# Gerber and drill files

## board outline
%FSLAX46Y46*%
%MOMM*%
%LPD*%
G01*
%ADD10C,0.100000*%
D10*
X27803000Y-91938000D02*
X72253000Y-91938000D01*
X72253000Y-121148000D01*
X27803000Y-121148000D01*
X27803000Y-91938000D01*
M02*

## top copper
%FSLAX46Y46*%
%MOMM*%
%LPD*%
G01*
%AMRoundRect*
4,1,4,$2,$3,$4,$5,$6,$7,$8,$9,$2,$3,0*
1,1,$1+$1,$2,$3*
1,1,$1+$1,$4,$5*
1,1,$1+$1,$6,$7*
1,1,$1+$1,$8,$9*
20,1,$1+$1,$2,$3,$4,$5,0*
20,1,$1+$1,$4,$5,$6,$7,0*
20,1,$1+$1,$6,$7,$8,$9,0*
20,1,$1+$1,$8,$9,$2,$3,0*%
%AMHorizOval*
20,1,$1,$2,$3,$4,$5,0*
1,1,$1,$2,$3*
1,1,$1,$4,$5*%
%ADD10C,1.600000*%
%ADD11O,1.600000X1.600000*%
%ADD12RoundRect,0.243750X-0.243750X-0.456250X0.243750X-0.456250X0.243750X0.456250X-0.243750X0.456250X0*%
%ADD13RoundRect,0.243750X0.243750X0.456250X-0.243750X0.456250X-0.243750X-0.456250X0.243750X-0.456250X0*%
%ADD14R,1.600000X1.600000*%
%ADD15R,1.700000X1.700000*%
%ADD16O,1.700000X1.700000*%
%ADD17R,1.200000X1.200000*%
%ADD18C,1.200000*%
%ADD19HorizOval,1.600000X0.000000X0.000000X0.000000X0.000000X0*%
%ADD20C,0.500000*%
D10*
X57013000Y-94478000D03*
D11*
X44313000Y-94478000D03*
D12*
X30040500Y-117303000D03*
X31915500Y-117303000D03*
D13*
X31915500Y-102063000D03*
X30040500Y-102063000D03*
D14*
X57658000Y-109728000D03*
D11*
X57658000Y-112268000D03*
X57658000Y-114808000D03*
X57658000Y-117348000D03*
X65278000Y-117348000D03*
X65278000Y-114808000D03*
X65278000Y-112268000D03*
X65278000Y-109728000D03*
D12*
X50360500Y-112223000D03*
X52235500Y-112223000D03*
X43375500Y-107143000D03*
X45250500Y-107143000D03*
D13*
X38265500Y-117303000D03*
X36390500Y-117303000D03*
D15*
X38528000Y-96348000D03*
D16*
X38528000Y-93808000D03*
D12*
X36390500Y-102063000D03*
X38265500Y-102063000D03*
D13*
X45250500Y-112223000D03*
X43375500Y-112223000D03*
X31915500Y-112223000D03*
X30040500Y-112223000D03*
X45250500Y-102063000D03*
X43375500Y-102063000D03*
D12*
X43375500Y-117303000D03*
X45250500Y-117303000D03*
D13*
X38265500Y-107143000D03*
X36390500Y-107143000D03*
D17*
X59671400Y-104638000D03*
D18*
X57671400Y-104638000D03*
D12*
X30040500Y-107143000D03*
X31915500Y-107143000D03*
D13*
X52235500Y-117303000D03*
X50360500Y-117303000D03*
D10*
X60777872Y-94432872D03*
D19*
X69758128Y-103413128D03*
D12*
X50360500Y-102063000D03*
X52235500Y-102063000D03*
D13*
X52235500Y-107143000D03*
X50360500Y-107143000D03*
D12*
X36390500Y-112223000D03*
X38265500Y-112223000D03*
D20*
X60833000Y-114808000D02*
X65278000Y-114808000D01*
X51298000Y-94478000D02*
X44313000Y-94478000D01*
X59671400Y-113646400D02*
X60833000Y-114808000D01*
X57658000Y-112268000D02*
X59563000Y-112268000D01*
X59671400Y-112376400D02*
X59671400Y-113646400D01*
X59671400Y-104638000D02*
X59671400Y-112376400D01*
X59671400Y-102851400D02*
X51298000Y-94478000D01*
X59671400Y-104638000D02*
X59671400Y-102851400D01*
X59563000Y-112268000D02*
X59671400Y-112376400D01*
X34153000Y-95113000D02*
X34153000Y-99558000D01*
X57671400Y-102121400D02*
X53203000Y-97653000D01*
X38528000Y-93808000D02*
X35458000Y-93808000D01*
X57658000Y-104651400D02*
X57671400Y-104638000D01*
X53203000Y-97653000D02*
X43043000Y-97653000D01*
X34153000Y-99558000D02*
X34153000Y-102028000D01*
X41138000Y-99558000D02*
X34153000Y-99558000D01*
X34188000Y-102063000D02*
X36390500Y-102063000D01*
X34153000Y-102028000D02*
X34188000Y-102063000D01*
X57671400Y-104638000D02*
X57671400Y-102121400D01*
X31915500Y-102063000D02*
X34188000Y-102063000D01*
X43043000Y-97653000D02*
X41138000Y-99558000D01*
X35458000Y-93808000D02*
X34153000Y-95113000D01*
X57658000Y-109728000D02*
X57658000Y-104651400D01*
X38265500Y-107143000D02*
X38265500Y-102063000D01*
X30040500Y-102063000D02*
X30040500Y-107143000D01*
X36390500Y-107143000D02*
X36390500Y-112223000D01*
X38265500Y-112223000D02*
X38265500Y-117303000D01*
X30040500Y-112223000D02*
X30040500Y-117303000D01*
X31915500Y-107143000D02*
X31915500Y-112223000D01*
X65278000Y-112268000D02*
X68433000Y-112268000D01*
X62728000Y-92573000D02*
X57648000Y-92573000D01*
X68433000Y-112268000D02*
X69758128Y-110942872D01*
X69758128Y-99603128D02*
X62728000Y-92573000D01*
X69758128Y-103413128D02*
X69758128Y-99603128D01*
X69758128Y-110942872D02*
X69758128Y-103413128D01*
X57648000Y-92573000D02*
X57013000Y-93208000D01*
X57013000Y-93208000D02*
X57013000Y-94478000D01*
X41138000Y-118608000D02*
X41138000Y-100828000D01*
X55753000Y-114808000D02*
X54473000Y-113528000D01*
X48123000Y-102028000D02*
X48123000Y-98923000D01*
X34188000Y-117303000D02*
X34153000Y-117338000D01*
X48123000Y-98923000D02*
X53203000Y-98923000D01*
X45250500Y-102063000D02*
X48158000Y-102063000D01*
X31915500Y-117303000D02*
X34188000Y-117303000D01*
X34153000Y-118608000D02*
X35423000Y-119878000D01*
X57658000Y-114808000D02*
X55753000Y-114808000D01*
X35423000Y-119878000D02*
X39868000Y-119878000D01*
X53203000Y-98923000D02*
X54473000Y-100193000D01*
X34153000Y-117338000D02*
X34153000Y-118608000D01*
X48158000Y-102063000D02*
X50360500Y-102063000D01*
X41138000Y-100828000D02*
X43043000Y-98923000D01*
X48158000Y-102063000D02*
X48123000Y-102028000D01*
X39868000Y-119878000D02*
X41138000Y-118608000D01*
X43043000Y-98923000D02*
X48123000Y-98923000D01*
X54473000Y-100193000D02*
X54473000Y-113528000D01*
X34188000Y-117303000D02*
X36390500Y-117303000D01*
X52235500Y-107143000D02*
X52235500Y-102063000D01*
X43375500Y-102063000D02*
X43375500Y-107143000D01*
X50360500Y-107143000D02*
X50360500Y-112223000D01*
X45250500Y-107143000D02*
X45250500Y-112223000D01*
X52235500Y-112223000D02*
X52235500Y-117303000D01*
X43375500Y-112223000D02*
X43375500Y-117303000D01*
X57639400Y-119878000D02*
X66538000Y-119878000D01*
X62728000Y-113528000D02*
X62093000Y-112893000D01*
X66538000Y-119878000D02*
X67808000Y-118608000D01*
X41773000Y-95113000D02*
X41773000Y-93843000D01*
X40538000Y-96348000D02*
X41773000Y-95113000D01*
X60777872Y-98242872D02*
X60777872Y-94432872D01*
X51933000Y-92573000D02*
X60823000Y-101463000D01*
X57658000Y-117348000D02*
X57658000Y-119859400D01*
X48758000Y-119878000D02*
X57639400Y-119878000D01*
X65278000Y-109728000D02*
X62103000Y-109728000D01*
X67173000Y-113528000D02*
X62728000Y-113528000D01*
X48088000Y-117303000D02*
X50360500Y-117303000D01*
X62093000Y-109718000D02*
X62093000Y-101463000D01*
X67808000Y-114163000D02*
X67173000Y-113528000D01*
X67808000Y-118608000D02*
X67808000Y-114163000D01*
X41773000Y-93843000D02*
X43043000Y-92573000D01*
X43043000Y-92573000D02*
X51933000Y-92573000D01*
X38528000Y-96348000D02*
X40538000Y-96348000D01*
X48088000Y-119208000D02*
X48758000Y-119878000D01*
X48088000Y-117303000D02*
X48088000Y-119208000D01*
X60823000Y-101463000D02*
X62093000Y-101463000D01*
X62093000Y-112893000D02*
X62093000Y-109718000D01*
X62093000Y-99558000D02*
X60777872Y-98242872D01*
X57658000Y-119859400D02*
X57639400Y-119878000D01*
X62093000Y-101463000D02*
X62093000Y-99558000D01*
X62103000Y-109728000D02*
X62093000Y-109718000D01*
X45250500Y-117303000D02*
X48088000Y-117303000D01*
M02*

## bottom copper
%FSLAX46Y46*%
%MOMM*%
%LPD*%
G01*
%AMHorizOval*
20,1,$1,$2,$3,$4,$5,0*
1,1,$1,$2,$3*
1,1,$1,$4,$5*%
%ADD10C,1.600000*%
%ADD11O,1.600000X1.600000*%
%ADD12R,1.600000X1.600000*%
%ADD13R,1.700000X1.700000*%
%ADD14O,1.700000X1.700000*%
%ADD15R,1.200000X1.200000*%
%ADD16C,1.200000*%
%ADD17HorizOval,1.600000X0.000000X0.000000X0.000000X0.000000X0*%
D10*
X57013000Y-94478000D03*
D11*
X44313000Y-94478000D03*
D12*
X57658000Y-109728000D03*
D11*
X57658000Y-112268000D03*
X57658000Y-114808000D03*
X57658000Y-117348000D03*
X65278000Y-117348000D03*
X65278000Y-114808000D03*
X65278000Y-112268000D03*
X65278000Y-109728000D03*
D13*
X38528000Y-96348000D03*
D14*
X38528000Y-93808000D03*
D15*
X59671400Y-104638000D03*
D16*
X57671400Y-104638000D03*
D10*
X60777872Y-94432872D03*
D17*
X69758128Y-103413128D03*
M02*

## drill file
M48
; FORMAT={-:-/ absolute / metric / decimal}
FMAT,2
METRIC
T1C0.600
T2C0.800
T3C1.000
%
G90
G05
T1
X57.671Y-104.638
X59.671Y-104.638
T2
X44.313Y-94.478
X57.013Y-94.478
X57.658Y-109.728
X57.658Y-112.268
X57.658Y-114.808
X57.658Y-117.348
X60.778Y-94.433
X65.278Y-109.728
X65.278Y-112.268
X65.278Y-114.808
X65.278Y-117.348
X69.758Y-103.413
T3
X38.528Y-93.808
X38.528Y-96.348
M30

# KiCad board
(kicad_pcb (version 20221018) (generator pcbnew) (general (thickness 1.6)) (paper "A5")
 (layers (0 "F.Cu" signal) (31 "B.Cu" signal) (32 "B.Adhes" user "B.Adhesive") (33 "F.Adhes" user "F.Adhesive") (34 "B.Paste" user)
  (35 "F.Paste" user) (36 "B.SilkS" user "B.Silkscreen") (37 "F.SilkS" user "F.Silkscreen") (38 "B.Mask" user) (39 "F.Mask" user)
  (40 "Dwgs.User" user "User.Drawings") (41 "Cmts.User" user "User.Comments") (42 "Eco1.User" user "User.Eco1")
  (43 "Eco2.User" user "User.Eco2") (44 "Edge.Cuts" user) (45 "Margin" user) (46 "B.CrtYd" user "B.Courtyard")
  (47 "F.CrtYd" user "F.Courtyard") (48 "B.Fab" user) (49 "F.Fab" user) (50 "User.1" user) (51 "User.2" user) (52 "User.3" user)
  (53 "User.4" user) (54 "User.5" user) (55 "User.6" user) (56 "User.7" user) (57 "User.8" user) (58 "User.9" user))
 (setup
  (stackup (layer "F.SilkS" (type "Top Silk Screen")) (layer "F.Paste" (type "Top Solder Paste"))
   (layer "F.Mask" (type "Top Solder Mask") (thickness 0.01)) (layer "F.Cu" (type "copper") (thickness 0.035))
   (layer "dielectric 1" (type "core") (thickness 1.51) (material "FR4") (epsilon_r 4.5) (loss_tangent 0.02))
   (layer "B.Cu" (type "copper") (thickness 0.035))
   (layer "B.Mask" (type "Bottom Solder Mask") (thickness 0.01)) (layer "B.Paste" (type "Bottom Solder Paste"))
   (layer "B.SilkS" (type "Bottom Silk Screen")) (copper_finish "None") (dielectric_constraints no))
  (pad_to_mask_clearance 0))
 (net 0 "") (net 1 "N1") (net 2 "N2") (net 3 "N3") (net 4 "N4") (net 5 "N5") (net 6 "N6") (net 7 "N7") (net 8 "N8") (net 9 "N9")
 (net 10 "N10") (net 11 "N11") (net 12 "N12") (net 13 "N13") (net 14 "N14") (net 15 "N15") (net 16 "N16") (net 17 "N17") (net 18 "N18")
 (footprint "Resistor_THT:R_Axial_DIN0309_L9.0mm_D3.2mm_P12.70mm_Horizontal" (layer "F.Cu") (at 57.013 94.478 180)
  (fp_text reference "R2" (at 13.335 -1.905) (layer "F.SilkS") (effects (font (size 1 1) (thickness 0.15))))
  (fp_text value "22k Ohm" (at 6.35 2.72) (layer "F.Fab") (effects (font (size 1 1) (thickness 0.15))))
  (pad "1" thru_hole circle (at 0 0 180) (size 1.6 1.6) (drill 0.8) (layers "*.Cu" "*.Mask") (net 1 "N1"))
  (pad "2" thru_hole oval (at 12.7 0 180) (size 1.6 1.6) (drill 0.8) (layers "*.Cu" "*.Mask") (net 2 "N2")))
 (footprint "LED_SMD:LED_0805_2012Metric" (layer "F.Cu") (at 30.978 117.303)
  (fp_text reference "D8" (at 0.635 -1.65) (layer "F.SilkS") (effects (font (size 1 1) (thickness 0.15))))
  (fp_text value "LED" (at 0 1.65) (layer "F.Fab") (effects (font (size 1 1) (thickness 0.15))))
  (pad "1" smd roundrect (at -0.9375 0) (size 0.975 1.4) (layers "F.Cu" "F.Paste" "F.Mask") (roundrect_rratio 0.25) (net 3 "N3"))
  (pad "2" smd roundrect (at 0.9375 0) (size 0.975 1.4) (layers "F.Cu" "F.Paste" "F.Mask") (roundrect_rratio 0.25) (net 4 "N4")))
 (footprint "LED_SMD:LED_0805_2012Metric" (layer "F.Cu") (at 30.978 102.063 180)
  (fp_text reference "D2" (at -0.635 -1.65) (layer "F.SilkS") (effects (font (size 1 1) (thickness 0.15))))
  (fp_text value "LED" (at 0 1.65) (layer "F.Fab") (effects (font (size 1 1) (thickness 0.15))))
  (pad "1" smd roundrect (at -0.9375 0 180) (size 0.975 1.4) (layers "F.Cu" "F.Paste" "F.Mask") (roundrect_rratio 0.25) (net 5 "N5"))
  (pad "2" smd roundrect (at 0.9375 0 180) (size 0.975 1.4) (layers "F.Cu" "F.Paste" "F.Mask") (roundrect_rratio 0.25) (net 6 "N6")))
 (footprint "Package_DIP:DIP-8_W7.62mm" (layer "F.Cu") (at 57.658 109.728)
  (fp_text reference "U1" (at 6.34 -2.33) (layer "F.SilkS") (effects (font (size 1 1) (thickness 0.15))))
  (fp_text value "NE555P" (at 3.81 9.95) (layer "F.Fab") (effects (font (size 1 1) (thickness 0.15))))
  (pad "1" thru_hole rect (at 0 0) (size 1.6 1.6) (drill 0.8) (layers "*.Cu" "*.Mask") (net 5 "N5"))
  (pad "2" thru_hole oval (at 0 2.54) (size 1.6 1.6) (drill 0.8) (layers "*.Cu" "*.Mask") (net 2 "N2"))
  (pad "3" thru_hole oval (at 0 5.08) (size 1.6 1.6) (drill 0.8) (layers "*.Cu" "*.Mask") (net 4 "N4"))
  (pad "4" thru_hole oval (at 0 7.62) (size 1.6 1.6) (drill 0.8) (layers "*.Cu" "*.Mask") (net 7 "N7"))
  (pad "5" thru_hole oval (at 7.62 7.62) (size 1.6 1.6) (drill 0.8) (layers "*.Cu" "*.Mask") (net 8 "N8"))
  (pad "6" thru_hole oval (at 7.62 5.08) (size 1.6 1.6) (drill 0.8) (layers "*.Cu" "*.Mask") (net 2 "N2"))
  (pad "7" thru_hole oval (at 7.62 2.54) (size 1.6 1.6) (drill 0.8) (layers "*.Cu" "*.Mask") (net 1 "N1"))
  (pad "8" thru_hole oval (at 7.62 0) (size 1.6 1.6) (drill 0.8) (layers "*.Cu" "*.Mask") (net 7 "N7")))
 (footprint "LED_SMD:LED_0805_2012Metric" (layer "F.Cu") (at 51.298 112.223)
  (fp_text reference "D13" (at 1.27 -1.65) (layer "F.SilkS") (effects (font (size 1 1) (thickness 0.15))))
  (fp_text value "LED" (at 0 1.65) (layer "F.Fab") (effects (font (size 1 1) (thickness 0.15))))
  (pad "1" smd roundrect (at -0.9375 0) (size 0.975 1.4) (layers "F.Cu" "F.Paste" "F.Mask") (roundrect_rratio 0.25) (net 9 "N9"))
  (pad "2" smd roundrect (at 0.9375 0) (size 0.975 1.4) (layers "F.Cu" "F.Paste" "F.Mask") (roundrect_rratio 0.25) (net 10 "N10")))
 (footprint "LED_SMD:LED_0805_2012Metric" (layer "F.Cu") (at 44.313 107.143)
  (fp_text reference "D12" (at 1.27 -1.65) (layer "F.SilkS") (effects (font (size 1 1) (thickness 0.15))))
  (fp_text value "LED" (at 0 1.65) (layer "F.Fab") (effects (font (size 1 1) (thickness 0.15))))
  (pad "1" smd roundrect (at -0.9375 0) (size 0.975 1.4) (layers "F.Cu" "F.Paste" "F.Mask") (roundrect_rratio 0.25) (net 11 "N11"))
  (pad "2" smd roundrect (at 0.9375 0) (size 0.975 1.4) (layers "F.Cu" "F.Paste" "F.Mask") (roundrect_rratio 0.25) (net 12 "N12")))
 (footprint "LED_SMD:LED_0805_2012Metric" (layer "F.Cu") (at 37.328 117.303 180)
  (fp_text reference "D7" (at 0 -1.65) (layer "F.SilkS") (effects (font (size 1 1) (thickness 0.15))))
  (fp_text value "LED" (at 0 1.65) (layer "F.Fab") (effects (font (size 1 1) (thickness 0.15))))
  (pad "1" smd roundrect (at -0.9375 0 180) (size 0.975 1.4) (layers "F.Cu" "F.Paste" "F.Mask") (roundrect_rratio 0.25) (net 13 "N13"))
  (pad "2" smd roundrect (at 0.9375 0 180) (size 0.975 1.4) (layers "F.Cu" "F.Paste" "F.Mask") (roundrect_rratio 0.25) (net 4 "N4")))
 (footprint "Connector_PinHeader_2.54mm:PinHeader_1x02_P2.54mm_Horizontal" (layer "F.Cu") (at 38.528 96.348 180)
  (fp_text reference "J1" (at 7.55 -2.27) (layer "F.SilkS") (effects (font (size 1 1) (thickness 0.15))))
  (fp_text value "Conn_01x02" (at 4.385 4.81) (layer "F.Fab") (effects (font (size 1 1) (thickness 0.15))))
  (pad "1" thru_hole rect (at 0 0 180) (size 1.7 1.7) (drill 1) (layers "*.Cu" "*.Mask") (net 7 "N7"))
  (pad "2" thru_hole oval (at 0 2.54 180) (size 1.7 1.7) (drill 1) (layers "*.Cu" "*.Mask") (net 5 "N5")))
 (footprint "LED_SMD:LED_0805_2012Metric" (layer "F.Cu") (at 37.328 102.063)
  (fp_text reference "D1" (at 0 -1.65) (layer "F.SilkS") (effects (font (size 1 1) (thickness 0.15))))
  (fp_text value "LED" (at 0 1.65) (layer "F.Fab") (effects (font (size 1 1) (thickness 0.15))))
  (pad "1" smd roundrect (at -0.9375 0) (size 0.975 1.4) (layers "F.Cu" "F.Paste" "F.Mask") (roundrect_rratio 0.25) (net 5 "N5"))
  (pad "2" smd roundrect (at 0.9375 0) (size 0.975 1.4) (layers "F.Cu" "F.Paste" "F.Mask") (roundrect_rratio 0.25) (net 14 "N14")))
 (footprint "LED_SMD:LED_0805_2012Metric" (layer "F.Cu") (at 44.313 112.223 180)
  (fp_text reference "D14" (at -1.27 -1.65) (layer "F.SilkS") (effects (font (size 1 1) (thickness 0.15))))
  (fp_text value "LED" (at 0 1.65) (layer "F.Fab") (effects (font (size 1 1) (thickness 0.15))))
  (pad "1" smd roundrect (at -0.9375 0 180) (size 0.975 1.4) (layers "F.Cu" "F.Paste" "F.Mask") (roundrect_rratio 0.25) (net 12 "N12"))
  (pad "2" smd roundrect (at 0.9375 0 180) (size 0.975 1.4) (layers "F.Cu" "F.Paste" "F.Mask") (roundrect_rratio 0.25) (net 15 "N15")))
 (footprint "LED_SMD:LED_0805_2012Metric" (layer "F.Cu") (at 30.978 112.223 180)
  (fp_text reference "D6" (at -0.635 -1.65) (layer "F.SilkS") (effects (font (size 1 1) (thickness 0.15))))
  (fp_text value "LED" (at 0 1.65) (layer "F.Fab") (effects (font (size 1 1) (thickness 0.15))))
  (pad "1" smd roundrect (at -0.9375 0 180) (size 0.975 1.4) (layers "F.Cu" "F.Paste" "F.Mask") (roundrect_rratio 0.25) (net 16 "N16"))
  (pad "2" smd roundrect (at 0.9375 0 180) (size 0.975 1.4) (layers "F.Cu" "F.Paste" "F.Mask") (roundrect_rratio 0.25) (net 3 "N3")))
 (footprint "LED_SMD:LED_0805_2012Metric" (layer "F.Cu") (at 44.313 102.063 180)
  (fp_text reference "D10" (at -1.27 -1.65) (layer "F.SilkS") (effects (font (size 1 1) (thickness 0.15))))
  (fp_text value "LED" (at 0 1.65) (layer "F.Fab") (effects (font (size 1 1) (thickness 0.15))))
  (pad "1" smd roundrect (at -0.9375 0 180) (size 0.975 1.4) (layers "F.Cu" "F.Paste" "F.Mask") (roundrect_rratio 0.25) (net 4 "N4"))
  (pad "2" smd roundrect (at 0.9375 0 180) (size 0.975 1.4) (layers "F.Cu" "F.Paste" "F.Mask") (roundrect_rratio 0.25) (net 11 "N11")))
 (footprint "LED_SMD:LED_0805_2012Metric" (layer "F.Cu") (at 44.313 117.303)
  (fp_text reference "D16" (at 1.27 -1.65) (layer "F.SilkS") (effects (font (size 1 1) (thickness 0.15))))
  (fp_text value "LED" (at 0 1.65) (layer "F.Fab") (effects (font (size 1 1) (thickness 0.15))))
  (pad "1" smd roundrect (at -0.9375 0) (size 0.975 1.4) (layers "F.Cu" "F.Paste" "F.Mask") (roundrect_rratio 0.25) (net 15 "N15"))
  (pad "2" smd roundrect (at 0.9375 0) (size 0.975 1.4) (layers "F.Cu" "F.Paste" "F.Mask") (roundrect_rratio 0.25) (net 7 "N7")))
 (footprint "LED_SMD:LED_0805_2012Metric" (layer "F.Cu") (at 37.328 107.143 180)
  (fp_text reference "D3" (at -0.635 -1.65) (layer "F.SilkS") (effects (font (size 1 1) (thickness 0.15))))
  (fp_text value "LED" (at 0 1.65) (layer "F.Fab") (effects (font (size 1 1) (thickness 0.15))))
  (pad "1" smd roundrect (at -0.9375 0 180) (size 0.975 1.4) (layers "F.Cu" "F.Paste" "F.Mask") (roundrect_rratio 0.25) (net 14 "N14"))
  (pad "2" smd roundrect (at 0.9375 0 180) (size 0.975 1.4) (layers "F.Cu" "F.Paste" "F.Mask") (roundrect_rratio 0.25) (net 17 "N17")))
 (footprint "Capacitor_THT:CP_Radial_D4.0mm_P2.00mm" (layer "F.Cu") (at 59.6714 104.638 180)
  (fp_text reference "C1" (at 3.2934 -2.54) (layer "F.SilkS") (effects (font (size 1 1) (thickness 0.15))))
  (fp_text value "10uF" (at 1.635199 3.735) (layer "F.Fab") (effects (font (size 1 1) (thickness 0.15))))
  (pad "1" thru_hole rect (at 0 0 180) (size 1.2 1.2) (drill 0.6) (layers "*.Cu" "*.Mask") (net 2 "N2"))
  (pad "2" thru_hole circle (at 2 0 180) (size 1.2 1.2) (drill 0.6) (layers "*.Cu" "*.Mask") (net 5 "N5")))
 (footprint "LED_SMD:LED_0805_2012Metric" (layer "F.Cu") (at 30.978 107.143)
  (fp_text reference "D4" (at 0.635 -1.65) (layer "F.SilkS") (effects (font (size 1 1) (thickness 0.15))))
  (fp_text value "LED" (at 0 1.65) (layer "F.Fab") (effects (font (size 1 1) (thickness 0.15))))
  (pad "1" smd roundrect (at -0.9375 0) (size 0.975 1.4) (layers "F.Cu" "F.Paste" "F.Mask") (roundrect_rratio 0.25) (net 6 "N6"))
  (pad "2" smd roundrect (at 0.9375 0) (size 0.975 1.4) (layers "F.Cu" "F.Paste" "F.Mask") (roundrect_rratio 0.25) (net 16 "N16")))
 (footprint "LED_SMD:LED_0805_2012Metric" (layer "F.Cu") (at 51.298 117.303 180)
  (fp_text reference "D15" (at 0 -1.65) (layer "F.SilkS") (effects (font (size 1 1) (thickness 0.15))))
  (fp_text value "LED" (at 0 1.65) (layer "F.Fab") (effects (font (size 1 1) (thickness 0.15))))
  (pad "1" smd roundrect (at -0.9375 0 180) (size 0.975 1.4) (layers "F.Cu" "F.Paste" "F.Mask") (roundrect_rratio 0.25) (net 10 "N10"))
  (pad "2" smd roundrect (at 0.9375 0 180) (size 0.975 1.4) (layers "F.Cu" "F.Paste" "F.Mask") (roundrect_rratio 0.25) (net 7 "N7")))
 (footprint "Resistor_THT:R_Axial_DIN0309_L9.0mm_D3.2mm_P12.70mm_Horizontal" (layer "F.Cu") (at 60.777872 94.432872 -45)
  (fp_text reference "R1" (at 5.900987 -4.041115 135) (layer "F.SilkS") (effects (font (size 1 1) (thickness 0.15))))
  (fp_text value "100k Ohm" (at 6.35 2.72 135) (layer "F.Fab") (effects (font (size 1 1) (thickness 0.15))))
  (pad "1" thru_hole circle (at 0 0 315) (size 1.6 1.6) (drill 0.8) (layers "*.Cu" "*.Mask") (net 7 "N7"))
  (pad "2" thru_hole oval (at 12.7 0 315) (size 1.6 1.6) (drill 0.8) (layers "*.Cu" "*.Mask") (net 1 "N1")))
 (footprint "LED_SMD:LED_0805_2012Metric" (layer "F.Cu") (at 51.298 102.063)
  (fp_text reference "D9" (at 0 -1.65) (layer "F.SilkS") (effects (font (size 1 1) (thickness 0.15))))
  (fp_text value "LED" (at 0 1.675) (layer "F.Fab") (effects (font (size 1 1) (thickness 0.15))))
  (pad "1" smd roundrect (at -0.9375 0) (size 0.975 1.4) (layers "F.Cu" "F.Paste" "F.Mask") (roundrect_rratio 0.25) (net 4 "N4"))
  (pad "2" smd roundrect (at 0.9375 0) (size 0.975 1.4) (layers "F.Cu" "F.Paste" "F.Mask") (roundrect_rratio 0.25) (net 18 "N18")))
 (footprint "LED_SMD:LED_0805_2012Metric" (layer "F.Cu") (at 51.298 107.143 180)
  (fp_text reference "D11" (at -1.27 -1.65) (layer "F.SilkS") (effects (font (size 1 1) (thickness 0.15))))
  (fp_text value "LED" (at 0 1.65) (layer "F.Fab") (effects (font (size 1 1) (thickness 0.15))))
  (pad "1" smd roundrect (at -0.9375 0 180) (size 0.975 1.4) (layers "F.Cu" "F.Paste" "F.Mask") (roundrect_rratio 0.25) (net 18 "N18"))
  (pad "2" smd roundrect (at 0.9375 0 180) (size 0.975 1.4) (layers "F.Cu" "F.Paste" "F.Mask") (roundrect_rratio 0.25) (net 9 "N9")))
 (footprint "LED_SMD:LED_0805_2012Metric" (layer "F.Cu") (at 37.328 112.223)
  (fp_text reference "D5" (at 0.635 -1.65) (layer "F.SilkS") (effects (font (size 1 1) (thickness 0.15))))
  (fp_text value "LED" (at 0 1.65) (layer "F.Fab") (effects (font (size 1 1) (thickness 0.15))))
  (pad "1" smd roundrect (at -0.9375 0) (size 0.975 1.4) (layers "F.Cu" "F.Paste" "F.Mask") (roundrect_rratio 0.25) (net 17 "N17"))
  (pad "2" smd roundrect (at 0.9375 0) (size 0.975 1.4) (layers "F.Cu" "F.Paste" "F.Mask") (roundrect_rratio 0.25) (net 13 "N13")))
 (gr_rect (start 27.803 91.938) (end 72.253 121.148) (stroke (width 0.1) (type solid)) (fill none) (layer "Edge.Cuts"))
 (segment (start 60.833 114.808) (end 65.278 114.808) (width 0.5) (layer "F.Cu") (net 2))
 (segment (start 51.298 94.478) (end 44.313 94.478) (width 0.5) (layer "F.Cu") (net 2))
 (segment (start 59.6714 113.6464) (end 60.833 114.808) (width 0.5) (layer "F.Cu") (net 2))
 (segment (start 57.658 112.268) (end 59.563 112.268) (width 0.5) (layer "F.Cu") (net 2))
 (segment (start 59.6714 112.3764) (end 59.6714 113.6464) (width 0.5) (layer "F.Cu") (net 2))
 (segment (start 59.6714 104.638) (end 59.6714 112.3764) (width 0.5) (layer "F.Cu") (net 2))
 (segment (start 59.6714 102.8514) (end 51.298 94.478) (width 0.5) (layer "F.Cu") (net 2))
 (segment (start 59.6714 104.638) (end 59.6714 102.8514) (width 0.5) (layer "F.Cu") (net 2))
 (segment (start 59.563 112.268) (end 59.6714 112.3764) (width 0.5) (layer "F.Cu") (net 2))
 (segment (start 34.153 95.113) (end 34.153 99.558) (width 0.5) (layer "F.Cu") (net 5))
 (segment (start 57.6714 102.1214) (end 53.203 97.653) (width 0.5) (layer "F.Cu") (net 5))
 (segment (start 38.528 93.808) (end 35.458 93.808) (width 0.5) (layer "F.Cu") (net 5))
 (segment (start 57.658 104.6514) (end 57.6714 104.638) (width 0.5) (layer "F.Cu") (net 5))
 (segment (start 53.203 97.653) (end 43.043 97.653) (width 0.5) (layer "F.Cu") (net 5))
 (segment (start 34.153 99.558) (end 34.153 102.028) (width 0.5) (layer "F.Cu") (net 5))
 (segment (start 41.138 99.558) (end 34.153 99.558) (width 0.5) (layer "F.Cu") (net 5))
 (segment (start 34.188 102.063) (end 36.3905 102.063) (width 0.5) (layer "F.Cu") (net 5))
 (segment (start 34.153 102.028) (end 34.188 102.063) (width 0.5) (layer "F.Cu") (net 5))
 (segment (start 57.6714 104.638) (end 57.6714 102.1214) (width 0.5) (layer "F.Cu") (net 5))
 (segment (start 31.9155 102.063) (end 34.188 102.063) (width 0.5) (layer "F.Cu") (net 5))
 (segment (start 43.043 97.653) (end 41.138 99.558) (width 0.5) (layer "F.Cu") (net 5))
 (segment (start 35.458 93.808) (end 34.153 95.113) (width 0.5) (layer "F.Cu") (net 5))
 (segment (start 57.658 109.728) (end 57.658 104.6514) (width 0.5) (layer "F.Cu") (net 5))
 (segment (start 38.2655 107.143) (end 38.2655 102.063) (width 0.5) (layer "F.Cu") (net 14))
 (segment (start 30.0405 102.063) (end 30.0405 107.143) (width 0.5) (layer "F.Cu") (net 6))
 (segment (start 36.3905 107.143) (end 36.3905 112.223) (width 0.5) (layer "F.Cu") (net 17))
 (segment (start 38.2655 112.223) (end 38.2655 117.303) (width 0.5) (layer "F.Cu") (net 13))
 (segment (start 30.0405 112.223) (end 30.0405 117.303) (width 0.5) (layer "F.Cu") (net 3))
 (segment (start 31.9155 107.143) (end 31.9155 112.223) (width 0.5) (layer "F.Cu") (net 16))
 (segment (start 65.278 112.268) (end 68.433 112.268) (width 0.5) (layer "F.Cu") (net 1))
 (segment (start 62.728 92.573) (end 57.648 92.573) (width 0.5) (layer "F.Cu") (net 1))
 (segment (start 68.433 112.268) (end 69.758128 110.942872) (width 0.5) (layer "F.Cu") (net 1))
 (segment (start 69.758128 99.603128) (end 62.728 92.573) (width 0.5) (layer "F.Cu") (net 1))
 (segment (start 69.758128 103.413128) (end 69.758128 99.603128) (width 0.5) (layer "F.Cu") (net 1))
 (segment (start 69.758128 110.942872) (end 69.758128 103.413128) (width 0.5) (layer "F.Cu") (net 1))
 (segment (start 57.648 92.573) (end 57.013 93.208) (width 0.5) (layer "F.Cu") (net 1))
 (segment (start 57.013 93.208) (end 57.013 94.478) (width 0.5) (layer "F.Cu") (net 1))
 (segment (start 41.138 118.608) (end 41.138 100.828) (width 0.5) (layer "F.Cu") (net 4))
 (segment (start 55.753 114.808) (end 54.473 113.528) (width 0.5) (layer "F.Cu") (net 4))
 (segment (start 48.123 102.028) (end 48.123 98.923) (width 0.5) (layer "F.Cu") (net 4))
 (segment (start 34.188 117.303) (end 34.153 117.338) (width 0.5) (layer "F.Cu") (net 4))
 (segment (start 48.123 98.923) (end 53.203 98.923) (width 0.5) (layer "F.Cu") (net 4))
 (segment (start 45.2505 102.063) (end 48.158 102.063) (width 0.5) (layer "F.Cu") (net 4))
 (segment (start 31.9155 117.303) (end 34.188 117.303) (width 0.5) (layer "F.Cu") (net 4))
 (segment (start 34.153 118.608) (end 35.423 119.878) (width 0.5) (layer "F.Cu") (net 4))
 (segment (start 57.658 114.808) (end 55.753 114.808) (width 0.5) (layer "F.Cu") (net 4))
 (segment (start 35.423 119.878) (end 39.868 119.878) (width 0.5) (layer "F.Cu") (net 4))
 (segment (start 53.203 98.923) (end 54.473 100.193) (width 0.5) (layer "F.Cu") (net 4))
 (segment (start 34.153 117.338) (end 34.153 118.608) (width 0.5) (layer "F.Cu") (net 4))
 (segment (start 48.158 102.063) (end 50.3605 102.063) (width 0.5) (layer "F.Cu") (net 4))
 (segment (start 41.138 100.828) (end 43.043 98.923) (width 0.5) (layer "F.Cu") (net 4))
 (segment (start 48.158 102.063) (end 48.123 102.028) (width 0.5) (layer "F.Cu") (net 4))
 (segment (start 39.868 119.878) (end 41.138 118.608) (width 0.5) (layer "F.Cu") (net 4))
 (segment (start 43.043 98.923) (end 48.123 98.923) (width 0.5) (layer "F.Cu") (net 4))
 (segment (start 54.473 100.193) (end 54.473 113.528) (width 0.5) (layer "F.Cu") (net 4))
 (segment (start 34.188 117.303) (end 36.3905 117.303) (width 0.5) (layer "F.Cu") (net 4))
 (segment (start 52.2355 107.143) (end 52.2355 102.063) (width 0.5) (layer "F.Cu") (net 18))
 (segment (start 43.3755 102.063) (end 43.3755 107.143) (width 0.5) (layer "F.Cu") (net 11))
 (segment (start 50.3605 107.143) (end 50.3605 112.223) (width 0.5) (layer "F.Cu") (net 9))
 (segment (start 45.2505 107.143) (end 45.2505 112.223) (width 0.5) (layer "F.Cu") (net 12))
 (segment (start 52.2355 112.223) (end 52.2355 117.303) (width 0.5) (layer "F.Cu") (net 10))
 (segment (start 43.3755 112.223) (end 43.3755 117.303) (width 0.5) (layer "F.Cu") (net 15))
 (segment (start 57.6394 119.878) (end 66.538 119.878) (width 0.5) (layer "F.Cu") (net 7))
 (segment (start 62.728 113.528) (end 62.093 112.893) (width 0.5) (layer "F.Cu") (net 7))
 (segment (start 66.538 119.878) (end 67.808 118.608) (width 0.5) (layer "F.Cu") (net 7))
 (segment (start 41.773 95.113) (end 41.773 93.843) (width 0.5) (layer "F.Cu") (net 7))
 (segment (start 40.538 96.348) (end 41.773 95.113) (width 0.5) (layer "F.Cu") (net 7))
 (segment (start 60.777872 98.242872) (end 60.777872 94.432872) (width 0.5) (layer "F.Cu") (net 7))
 (segment (start 51.933 92.573) (end 60.823 101.463) (width 0.5) (layer "F.Cu") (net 7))
 (segment (start 57.658 117.348) (end 57.658 119.8594) (width 0.5) (layer "F.Cu") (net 7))
 (segment (start 48.758 119.878) (end 57.6394 119.878) (width 0.5) (layer "F.Cu") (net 7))
 (segment (start 65.278 109.728) (end 62.103 109.728) (width 0.5) (layer "F.Cu") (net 7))
 (segment (start 67.173 113.528) (end 62.728 113.528) (width 0.5) (layer "F.Cu") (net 7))
 (segment (start 48.088 117.303) (end 50.3605 117.303) (width 0.5) (layer "F.Cu") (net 7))
 (segment (start 62.093 109.718) (end 62.093 101.463) (width 0.5) (layer "F.Cu") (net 7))
 (segment (start 67.808 114.163) (end 67.173 113.528) (width 0.5) (layer "F.Cu") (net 7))
 (segment (start 67.808 118.608) (end 67.808 114.163) (width 0.5) (layer "F.Cu") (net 7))
 (segment (start 41.773 93.843) (end 43.043 92.573) (width 0.5) (layer "F.Cu") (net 7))
 (segment (start 43.043 92.573) (end 51.933 92.573) (width 0.5) (layer "F.Cu") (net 7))
 (segment (start 38.528 96.348) (end 40.538 96.348) (width 0.5) (layer "F.Cu") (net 7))
 (segment (start 48.088 119.208) (end 48.758 119.878) (width 0.5) (layer "F.Cu") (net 7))
 (segment (start 48.088 117.303) (end 48.088 119.208) (width 0.5) (layer "F.Cu") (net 7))
 (segment (start 60.823 101.463) (end 62.093 101.463) (width 0.5) (layer "F.Cu") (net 7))
 (segment (start 62.093 112.893) (end 62.093 109.718) (width 0.5) (layer "F.Cu") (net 7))
 (segment (start 62.093 99.558) (end 60.777872 98.242872) (width 0.5) (layer "F.Cu") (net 7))
 (segment (start 57.658 119.8594) (end 57.6394 119.878) (width 0.5) (layer "F.Cu") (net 7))
 (segment (start 62.093 101.463) (end 62.093 99.558) (width 0.5) (layer "F.Cu") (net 7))
 (segment (start 62.103 109.728) (end 62.093 109.718) (width 0.5) (layer "F.Cu") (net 7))
 (segment (start 45.2505 117.303) (end 48.088 117.303) (width 0.5) (layer "F.Cu") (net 7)))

